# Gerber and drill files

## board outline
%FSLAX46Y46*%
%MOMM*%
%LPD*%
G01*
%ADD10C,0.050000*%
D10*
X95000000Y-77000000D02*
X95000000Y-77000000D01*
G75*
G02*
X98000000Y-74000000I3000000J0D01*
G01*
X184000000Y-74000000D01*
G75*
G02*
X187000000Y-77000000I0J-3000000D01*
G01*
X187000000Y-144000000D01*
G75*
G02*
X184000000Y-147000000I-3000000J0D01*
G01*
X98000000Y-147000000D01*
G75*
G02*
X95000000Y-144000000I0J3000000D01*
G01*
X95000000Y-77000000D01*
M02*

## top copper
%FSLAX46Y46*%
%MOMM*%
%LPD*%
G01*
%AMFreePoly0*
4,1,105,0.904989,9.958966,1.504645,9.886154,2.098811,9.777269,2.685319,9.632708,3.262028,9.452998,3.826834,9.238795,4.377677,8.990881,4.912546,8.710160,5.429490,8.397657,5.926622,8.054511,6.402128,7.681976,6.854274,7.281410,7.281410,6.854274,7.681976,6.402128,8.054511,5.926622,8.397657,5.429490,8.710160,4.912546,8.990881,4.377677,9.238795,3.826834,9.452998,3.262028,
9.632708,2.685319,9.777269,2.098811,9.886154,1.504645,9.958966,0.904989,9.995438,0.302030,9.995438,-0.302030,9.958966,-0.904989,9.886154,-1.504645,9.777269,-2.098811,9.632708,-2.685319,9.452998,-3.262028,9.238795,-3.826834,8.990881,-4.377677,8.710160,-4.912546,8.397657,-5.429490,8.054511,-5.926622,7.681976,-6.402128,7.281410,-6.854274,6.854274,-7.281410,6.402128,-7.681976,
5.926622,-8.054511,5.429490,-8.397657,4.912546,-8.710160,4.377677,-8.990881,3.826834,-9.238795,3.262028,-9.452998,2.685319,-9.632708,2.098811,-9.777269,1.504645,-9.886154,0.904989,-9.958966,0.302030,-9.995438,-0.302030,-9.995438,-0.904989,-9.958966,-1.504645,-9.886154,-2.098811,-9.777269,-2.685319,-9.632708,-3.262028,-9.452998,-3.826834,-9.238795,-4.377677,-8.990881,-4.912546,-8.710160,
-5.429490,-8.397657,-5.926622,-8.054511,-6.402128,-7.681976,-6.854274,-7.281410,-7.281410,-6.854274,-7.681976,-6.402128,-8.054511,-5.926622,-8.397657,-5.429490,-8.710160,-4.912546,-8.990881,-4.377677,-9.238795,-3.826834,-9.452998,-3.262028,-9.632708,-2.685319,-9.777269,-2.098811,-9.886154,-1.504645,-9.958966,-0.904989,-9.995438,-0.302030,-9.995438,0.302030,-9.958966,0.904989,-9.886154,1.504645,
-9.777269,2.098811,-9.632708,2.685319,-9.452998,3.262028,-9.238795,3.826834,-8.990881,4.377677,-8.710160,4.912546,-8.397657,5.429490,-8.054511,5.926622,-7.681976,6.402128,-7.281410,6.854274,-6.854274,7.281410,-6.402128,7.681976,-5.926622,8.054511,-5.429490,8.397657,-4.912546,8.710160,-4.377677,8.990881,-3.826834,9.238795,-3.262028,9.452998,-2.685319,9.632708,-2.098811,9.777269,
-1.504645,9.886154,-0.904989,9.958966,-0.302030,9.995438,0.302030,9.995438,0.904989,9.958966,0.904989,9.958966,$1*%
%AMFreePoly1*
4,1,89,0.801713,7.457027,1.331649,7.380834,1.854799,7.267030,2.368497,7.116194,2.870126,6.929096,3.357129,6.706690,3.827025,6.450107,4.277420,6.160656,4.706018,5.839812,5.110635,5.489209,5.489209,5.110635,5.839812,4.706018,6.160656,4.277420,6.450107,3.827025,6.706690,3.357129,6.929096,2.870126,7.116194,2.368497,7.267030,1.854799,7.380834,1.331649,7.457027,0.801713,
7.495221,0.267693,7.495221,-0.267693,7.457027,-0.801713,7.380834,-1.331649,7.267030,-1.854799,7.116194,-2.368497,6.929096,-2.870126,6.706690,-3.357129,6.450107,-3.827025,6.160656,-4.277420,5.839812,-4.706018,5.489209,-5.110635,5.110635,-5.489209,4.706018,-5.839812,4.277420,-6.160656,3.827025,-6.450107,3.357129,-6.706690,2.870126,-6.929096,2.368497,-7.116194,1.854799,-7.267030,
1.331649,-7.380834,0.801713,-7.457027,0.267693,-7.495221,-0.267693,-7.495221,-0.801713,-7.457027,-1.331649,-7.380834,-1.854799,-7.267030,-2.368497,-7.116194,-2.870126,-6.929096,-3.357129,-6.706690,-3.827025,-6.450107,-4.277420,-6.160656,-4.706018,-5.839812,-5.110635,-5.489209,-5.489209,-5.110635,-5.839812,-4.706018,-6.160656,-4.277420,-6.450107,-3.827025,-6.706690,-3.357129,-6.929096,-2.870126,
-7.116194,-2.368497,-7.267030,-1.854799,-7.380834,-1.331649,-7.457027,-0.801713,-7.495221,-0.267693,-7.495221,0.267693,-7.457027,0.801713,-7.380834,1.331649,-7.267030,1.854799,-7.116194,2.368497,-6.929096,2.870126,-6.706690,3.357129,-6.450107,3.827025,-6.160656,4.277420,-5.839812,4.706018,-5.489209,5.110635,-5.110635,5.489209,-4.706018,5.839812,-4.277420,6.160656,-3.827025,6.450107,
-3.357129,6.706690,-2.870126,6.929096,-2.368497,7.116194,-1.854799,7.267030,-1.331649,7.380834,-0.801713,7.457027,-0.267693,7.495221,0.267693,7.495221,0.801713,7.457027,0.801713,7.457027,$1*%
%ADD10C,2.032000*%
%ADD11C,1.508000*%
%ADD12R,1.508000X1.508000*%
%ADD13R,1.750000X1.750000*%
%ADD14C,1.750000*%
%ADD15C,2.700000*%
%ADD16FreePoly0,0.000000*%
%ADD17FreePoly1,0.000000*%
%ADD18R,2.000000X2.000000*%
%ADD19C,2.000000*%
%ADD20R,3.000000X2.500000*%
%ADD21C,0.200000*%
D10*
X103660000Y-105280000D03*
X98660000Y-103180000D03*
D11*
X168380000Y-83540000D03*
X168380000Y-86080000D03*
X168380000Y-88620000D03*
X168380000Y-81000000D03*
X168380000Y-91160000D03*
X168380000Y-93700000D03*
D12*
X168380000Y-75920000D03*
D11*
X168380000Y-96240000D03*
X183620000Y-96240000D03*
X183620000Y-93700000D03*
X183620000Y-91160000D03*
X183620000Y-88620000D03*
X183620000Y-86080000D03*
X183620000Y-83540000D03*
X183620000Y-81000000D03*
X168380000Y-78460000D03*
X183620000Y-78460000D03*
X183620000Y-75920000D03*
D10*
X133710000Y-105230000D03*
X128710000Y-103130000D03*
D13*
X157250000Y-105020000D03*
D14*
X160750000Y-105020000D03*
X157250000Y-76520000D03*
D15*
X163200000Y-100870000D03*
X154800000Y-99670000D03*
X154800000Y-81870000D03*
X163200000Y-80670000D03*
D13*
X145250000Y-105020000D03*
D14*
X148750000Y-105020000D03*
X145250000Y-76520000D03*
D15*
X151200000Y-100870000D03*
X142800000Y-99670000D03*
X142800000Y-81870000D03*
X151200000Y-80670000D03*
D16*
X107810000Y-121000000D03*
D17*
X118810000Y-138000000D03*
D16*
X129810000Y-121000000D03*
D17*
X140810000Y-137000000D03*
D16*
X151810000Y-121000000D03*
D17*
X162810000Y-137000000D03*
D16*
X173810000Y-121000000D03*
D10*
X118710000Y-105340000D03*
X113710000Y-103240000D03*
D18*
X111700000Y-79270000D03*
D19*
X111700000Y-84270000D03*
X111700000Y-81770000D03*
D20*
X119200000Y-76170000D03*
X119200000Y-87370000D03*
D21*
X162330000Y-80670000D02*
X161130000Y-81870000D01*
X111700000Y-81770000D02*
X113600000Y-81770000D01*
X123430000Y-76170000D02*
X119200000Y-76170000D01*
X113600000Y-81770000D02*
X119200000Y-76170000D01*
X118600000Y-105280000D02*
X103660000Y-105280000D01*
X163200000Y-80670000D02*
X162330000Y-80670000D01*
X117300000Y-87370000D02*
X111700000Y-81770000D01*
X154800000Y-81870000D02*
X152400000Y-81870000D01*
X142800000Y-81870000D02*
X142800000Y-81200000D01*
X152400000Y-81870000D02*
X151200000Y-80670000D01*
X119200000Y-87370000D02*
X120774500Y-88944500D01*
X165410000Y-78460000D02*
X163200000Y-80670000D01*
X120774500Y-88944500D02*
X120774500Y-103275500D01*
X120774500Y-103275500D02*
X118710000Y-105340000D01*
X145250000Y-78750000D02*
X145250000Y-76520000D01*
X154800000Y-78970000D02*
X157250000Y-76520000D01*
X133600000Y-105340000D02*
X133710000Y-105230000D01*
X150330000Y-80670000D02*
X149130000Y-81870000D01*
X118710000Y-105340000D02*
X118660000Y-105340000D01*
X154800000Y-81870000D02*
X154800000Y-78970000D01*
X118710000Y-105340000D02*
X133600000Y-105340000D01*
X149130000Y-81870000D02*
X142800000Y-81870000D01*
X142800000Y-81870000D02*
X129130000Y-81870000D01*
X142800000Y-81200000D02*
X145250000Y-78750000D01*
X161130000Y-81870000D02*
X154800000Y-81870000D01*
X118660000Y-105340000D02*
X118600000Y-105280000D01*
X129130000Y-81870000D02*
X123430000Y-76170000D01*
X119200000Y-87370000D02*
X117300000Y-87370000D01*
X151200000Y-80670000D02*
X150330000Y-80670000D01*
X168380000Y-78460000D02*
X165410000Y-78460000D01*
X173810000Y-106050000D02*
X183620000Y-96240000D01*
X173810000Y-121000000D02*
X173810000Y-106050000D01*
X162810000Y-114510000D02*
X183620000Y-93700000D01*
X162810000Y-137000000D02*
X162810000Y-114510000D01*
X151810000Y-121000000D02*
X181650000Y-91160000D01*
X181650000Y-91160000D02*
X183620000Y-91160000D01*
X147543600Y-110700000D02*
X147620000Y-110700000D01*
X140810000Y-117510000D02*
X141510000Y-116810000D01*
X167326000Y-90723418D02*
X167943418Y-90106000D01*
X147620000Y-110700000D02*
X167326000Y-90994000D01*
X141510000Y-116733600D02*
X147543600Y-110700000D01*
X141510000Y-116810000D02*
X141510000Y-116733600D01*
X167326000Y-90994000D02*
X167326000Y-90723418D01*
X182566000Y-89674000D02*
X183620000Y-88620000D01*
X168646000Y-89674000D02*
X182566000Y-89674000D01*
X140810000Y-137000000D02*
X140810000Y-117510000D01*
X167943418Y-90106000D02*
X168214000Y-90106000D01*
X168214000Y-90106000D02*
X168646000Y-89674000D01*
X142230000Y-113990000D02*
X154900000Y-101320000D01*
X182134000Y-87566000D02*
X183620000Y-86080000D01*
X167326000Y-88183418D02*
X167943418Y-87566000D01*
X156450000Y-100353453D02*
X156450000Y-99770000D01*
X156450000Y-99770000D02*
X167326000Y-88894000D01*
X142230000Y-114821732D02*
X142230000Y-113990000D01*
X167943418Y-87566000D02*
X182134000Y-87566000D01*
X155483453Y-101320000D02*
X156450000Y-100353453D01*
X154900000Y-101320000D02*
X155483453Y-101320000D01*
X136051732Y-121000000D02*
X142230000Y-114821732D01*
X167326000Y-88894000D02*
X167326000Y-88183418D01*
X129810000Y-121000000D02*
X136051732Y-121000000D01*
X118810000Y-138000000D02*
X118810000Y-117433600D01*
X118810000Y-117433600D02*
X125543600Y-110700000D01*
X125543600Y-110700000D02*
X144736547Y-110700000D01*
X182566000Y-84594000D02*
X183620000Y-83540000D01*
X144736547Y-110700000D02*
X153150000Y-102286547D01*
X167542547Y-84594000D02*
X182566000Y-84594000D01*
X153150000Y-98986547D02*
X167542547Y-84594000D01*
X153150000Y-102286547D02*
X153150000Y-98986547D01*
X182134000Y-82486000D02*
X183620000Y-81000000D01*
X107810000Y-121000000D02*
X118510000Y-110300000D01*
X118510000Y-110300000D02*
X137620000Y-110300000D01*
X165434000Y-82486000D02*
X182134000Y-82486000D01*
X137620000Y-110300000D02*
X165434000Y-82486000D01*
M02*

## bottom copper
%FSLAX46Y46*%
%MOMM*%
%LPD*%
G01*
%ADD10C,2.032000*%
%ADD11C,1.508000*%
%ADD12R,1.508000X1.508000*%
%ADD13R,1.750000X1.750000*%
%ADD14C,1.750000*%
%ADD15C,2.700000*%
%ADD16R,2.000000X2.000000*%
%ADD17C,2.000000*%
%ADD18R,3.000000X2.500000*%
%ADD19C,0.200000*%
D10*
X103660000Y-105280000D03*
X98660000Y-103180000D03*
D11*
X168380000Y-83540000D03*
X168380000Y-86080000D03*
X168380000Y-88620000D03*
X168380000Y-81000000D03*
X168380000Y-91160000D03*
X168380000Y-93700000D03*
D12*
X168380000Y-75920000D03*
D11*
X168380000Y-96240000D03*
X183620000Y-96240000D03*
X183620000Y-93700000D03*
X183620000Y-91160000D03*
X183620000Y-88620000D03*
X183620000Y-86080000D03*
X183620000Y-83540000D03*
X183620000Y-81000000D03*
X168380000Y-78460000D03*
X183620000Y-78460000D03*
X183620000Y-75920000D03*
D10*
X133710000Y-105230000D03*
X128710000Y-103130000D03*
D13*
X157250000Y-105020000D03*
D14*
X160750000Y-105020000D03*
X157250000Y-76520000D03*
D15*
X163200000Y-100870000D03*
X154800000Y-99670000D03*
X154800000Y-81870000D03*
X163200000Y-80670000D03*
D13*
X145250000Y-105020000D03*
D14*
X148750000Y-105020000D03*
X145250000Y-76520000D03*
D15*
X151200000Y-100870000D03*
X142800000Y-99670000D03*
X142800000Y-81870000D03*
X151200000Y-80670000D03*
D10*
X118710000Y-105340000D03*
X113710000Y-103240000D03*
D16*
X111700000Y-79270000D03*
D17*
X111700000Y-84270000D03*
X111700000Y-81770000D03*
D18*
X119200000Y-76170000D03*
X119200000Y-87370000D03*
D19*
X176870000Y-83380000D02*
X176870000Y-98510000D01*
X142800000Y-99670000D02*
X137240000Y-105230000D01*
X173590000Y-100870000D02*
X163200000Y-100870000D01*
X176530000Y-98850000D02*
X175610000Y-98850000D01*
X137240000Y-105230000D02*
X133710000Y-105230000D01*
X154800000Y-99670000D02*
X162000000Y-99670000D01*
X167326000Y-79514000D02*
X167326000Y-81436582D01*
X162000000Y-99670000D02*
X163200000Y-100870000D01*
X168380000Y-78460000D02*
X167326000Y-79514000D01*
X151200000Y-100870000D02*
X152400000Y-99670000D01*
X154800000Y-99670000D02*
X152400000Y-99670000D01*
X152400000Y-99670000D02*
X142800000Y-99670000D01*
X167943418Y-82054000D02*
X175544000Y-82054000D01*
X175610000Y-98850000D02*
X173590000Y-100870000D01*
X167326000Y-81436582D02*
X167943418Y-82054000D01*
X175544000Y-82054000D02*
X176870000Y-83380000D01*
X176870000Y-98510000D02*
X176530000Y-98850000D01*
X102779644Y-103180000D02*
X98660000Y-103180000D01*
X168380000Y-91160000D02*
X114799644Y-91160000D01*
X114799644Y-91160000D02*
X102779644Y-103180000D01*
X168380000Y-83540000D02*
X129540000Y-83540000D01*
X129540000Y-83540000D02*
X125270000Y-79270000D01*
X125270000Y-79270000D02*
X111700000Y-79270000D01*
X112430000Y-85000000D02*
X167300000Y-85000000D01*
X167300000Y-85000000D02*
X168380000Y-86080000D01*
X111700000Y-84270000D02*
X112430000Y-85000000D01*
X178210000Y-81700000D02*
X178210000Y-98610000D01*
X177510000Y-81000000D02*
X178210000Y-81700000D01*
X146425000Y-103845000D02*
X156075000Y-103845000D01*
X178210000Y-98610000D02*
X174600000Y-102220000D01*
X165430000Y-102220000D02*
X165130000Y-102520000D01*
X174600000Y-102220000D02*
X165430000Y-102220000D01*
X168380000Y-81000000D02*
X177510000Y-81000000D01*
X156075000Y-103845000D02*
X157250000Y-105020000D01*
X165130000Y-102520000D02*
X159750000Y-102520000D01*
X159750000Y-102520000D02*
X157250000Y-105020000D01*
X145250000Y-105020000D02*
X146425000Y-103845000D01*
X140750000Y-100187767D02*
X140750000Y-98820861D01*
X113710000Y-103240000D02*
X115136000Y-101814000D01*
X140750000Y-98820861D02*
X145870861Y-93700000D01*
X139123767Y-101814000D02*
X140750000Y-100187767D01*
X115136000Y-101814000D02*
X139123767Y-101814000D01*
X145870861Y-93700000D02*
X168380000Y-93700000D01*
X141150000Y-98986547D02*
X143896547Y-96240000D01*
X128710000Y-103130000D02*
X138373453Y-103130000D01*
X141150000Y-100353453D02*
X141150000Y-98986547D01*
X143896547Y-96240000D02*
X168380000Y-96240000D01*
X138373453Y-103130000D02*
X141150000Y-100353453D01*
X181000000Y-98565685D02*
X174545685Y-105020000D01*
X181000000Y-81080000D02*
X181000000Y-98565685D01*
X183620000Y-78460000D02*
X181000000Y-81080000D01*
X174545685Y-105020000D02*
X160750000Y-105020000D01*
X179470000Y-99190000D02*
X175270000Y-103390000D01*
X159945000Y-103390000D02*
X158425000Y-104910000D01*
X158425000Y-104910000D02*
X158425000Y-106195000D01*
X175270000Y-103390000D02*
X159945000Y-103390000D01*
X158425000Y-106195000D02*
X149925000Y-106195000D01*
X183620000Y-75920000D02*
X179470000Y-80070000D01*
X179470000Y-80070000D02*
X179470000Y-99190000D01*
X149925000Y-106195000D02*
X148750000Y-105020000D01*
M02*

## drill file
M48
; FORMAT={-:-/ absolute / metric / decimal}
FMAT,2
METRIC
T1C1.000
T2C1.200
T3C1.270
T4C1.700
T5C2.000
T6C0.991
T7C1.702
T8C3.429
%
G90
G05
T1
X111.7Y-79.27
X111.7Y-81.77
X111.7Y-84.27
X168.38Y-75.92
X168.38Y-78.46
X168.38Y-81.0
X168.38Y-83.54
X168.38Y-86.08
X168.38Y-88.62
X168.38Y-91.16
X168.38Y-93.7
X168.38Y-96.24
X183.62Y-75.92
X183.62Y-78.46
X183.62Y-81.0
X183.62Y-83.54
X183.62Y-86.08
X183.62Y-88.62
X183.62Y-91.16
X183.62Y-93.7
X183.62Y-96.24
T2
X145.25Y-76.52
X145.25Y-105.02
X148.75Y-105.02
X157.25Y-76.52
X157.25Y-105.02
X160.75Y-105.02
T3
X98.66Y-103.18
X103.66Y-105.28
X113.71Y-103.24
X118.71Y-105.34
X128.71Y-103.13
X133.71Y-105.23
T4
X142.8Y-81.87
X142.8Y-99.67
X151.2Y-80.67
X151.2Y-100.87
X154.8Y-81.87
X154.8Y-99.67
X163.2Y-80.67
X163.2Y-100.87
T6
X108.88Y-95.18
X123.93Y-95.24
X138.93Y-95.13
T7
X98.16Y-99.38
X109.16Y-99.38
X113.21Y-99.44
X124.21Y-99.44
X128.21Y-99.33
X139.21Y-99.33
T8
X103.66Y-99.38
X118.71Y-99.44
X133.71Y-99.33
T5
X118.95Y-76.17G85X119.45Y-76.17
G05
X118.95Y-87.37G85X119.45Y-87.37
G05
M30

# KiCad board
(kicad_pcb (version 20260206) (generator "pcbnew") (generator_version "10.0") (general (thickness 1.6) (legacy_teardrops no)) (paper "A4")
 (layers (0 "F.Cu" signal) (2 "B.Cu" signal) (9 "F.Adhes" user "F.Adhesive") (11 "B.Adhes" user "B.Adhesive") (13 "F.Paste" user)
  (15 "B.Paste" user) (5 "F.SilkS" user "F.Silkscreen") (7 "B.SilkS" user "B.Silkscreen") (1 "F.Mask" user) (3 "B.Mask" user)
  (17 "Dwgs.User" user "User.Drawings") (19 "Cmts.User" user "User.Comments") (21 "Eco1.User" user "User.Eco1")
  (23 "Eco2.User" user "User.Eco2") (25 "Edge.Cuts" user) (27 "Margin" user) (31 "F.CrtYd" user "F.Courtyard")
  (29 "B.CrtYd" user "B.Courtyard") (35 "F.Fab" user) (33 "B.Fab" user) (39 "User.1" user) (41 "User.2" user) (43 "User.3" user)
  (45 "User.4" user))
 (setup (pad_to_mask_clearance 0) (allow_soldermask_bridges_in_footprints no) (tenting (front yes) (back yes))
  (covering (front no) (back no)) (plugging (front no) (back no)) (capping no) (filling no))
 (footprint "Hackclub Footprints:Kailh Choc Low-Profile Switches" (layer "F.Cu") (at 103.66 99.38)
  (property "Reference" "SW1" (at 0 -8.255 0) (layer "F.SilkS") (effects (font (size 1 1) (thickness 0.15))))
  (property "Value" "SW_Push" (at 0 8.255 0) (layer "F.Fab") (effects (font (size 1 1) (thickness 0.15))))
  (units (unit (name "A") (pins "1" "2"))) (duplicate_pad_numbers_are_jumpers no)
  (pad "" np_thru_hole circle (at -5.5 0) (size 1.7018 1.7018) (drill 1.7018) (layers "*.Cu" "*.Mask"))
  (pad "" np_thru_hole circle (at 0 0) (size 3.429 3.429) (drill 3.429) (layers "*.Cu" "*.Mask"))
  (pad "" np_thru_hole circle (at 5.22 -4.2) (size 0.9906 0.9906) (drill 0.9906) (layers "*.Cu" "*.Mask"))
  (pad "" np_thru_hole circle (at 5.5 0) (size 1.7018 1.7018) (drill 1.7018) (layers "*.Cu" "*.Mask"))
  (pad "1" thru_hole circle (at 0 5.9) (size 2.032 2.032) (drill 1.27) (layers "*.Cu" "*.Mask") (remove_unused_layers no) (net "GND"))
  (pad "2" thru_hole circle (at -5 3.8) (size 2.032 2.032) (drill 1.27) (layers "*.Cu" "*.Mask") (remove_unused_layers no) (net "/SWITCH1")))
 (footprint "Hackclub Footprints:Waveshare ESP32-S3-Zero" (layer "F.Cu") (at 176 86.08)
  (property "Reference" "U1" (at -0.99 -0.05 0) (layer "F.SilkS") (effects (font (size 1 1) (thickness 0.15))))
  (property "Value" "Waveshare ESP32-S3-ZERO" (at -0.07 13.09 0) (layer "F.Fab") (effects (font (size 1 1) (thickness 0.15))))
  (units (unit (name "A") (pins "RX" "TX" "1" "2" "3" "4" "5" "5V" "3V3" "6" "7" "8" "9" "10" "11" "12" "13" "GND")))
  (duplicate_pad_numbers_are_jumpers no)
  (pad "1" thru_hole circle (at -7.62 -2.54) (size 1.508 1.508) (drill 1) (layers "*.Cu" "*.Mask") (remove_unused_layers no) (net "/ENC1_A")
   (solder_mask_margin 0.102))
  (pad "2" thru_hole circle (at -7.62 0) (size 1.508 1.508) (drill 1) (layers "*.Cu" "*.Mask") (remove_unused_layers no) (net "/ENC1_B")
   (solder_mask_margin 0.102))
  (pad "3" thru_hole circle (at -7.62 2.54) (size 1.508 1.508) (drill 1) (layers "*.Cu" "*.Mask") (remove_unused_layers no)
   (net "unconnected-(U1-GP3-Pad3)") (solder_mask_margin 0.102))
  (pad "3V3" thru_hole circle (at -7.62 -5.08) (size 1.508 1.508) (drill 1) (layers "*.Cu" "*.Mask") (remove_unused_layers no) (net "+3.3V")
   (solder_mask_margin 0.102))
  (pad "4" thru_hole circle (at -7.62 5.08) (size 1.508 1.508) (drill 1) (layers "*.Cu" "*.Mask") (remove_unused_layers no) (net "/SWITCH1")
   (solder_mask_margin 0.102))
  (pad "5" thru_hole circle (at -7.62 7.62) (size 1.508 1.508) (drill 1) (layers "*.Cu" "*.Mask") (remove_unused_layers no) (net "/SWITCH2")
   (solder_mask_margin 0.102))
  (pad "5V" thru_hole rect (at -7.62 -10.16) (size 1.508 1.508) (drill 1) (layers "*.Cu" "*.Mask") (remove_unused_layers no) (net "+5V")
   (solder_mask_margin 0.102))
  (pad "6" thru_hole circle (at -7.62 10.16) (size 1.508 1.508) (drill 1) (layers "*.Cu" "*.Mask") (remove_unused_layers no)
   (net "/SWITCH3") (solder_mask_margin 0.102))
  (pad "7" thru_hole circle (at 7.62 10.16) (size 1.508 1.508) (drill 1) (layers "*.Cu" "*.Mask") (remove_unused_layers no) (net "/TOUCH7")
   (solder_mask_margin 0.102))
  (pad "8" thru_hole circle (at 7.62 7.62) (size 1.508 1.508) (drill 1) (layers "*.Cu" "*.Mask") (remove_unused_layers no) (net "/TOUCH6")
   (solder_mask_margin 0.102))
  (pad "9" thru_hole circle (at 7.62 5.08) (size 1.508 1.508) (drill 1) (layers "*.Cu" "*.Mask") (remove_unused_layers no) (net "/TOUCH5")
   (solder_mask_margin 0.102))
  (pad "10" thru_hole circle (at 7.62 2.54) (size 1.508 1.508) (drill 1) (layers "*.Cu" "*.Mask") (remove_unused_layers no) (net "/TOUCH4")
   (solder_mask_margin 0.102))
  (pad "11" thru_hole circle (at 7.62 0) (size 1.508 1.508) (drill 1) (layers "*.Cu" "*.Mask") (remove_unused_layers no) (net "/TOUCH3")
   (solder_mask_margin 0.102))
  (pad "12" thru_hole circle (at 7.62 -2.54) (size 1.508 1.508) (drill 1) (layers "*.Cu" "*.Mask") (remove_unused_layers no) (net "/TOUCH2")
   (solder_mask_margin 0.102))
  (pad "13" thru_hole circle (at 7.62 -5.08) (size 1.508 1.508) (drill 1) (layers "*.Cu" "*.Mask") (remove_unused_layers no) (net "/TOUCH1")
   (solder_mask_margin 0.102))
  (pad "GND" thru_hole circle (at -7.62 -7.62) (size 1.508 1.508) (drill 1) (layers "*.Cu" "*.Mask") (remove_unused_layers no) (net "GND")
   (solder_mask_margin 0.102))
  (pad "RX" thru_hole circle (at 7.62 -7.62) (size 1.508 1.508) (drill 1) (layers "*.Cu" "*.Mask") (remove_unused_layers no)
   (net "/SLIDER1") (solder_mask_margin 0.102))
  (pad "TX" thru_hole circle (at 7.62 -10.16) (size 1.508 1.508) (drill 1) (layers "*.Cu" "*.Mask") (remove_unused_layers no)
   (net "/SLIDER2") (solder_mask_margin 0.102)))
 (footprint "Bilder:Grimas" (layer "F.Cu") (at 102.615412 81.967533)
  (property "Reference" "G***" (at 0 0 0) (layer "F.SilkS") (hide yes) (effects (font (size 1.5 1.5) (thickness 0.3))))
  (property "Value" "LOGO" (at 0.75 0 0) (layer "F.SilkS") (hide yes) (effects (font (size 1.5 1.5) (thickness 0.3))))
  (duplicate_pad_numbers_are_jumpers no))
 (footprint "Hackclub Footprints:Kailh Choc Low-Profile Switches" (layer "F.Cu") (at 133.71 99.33)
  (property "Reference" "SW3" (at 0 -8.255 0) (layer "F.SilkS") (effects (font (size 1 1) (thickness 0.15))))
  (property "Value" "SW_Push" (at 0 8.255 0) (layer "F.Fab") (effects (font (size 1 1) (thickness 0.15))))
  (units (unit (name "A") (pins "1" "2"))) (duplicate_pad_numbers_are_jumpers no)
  (pad "" np_thru_hole circle (at -5.5 0) (size 1.7018 1.7018) (drill 1.7018) (layers "*.Cu" "*.Mask"))
  (pad "" np_thru_hole circle (at 0 0) (size 3.429 3.429) (drill 3.429) (layers "*.Cu" "*.Mask"))
  (pad "" np_thru_hole circle (at 5.22 -4.2) (size 0.9906 0.9906) (drill 0.9906) (layers "*.Cu" "*.Mask"))
  (pad "" np_thru_hole circle (at 5.5 0) (size 1.7018 1.7018) (drill 1.7018) (layers "*.Cu" "*.Mask"))
  (pad "1" thru_hole circle (at 0 5.9) (size 2.032 2.032) (drill 1.27) (layers "*.Cu" "*.Mask") (remove_unused_layers no) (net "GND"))
  (pad "2" thru_hole circle (at -5 3.8) (size 2.032 2.032) (drill 1.27) (layers "*.Cu" "*.Mask") (remove_unused_layers no) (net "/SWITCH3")))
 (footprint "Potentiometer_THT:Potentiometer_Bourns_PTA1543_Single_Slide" (layer "F.Cu") (at 157.25 105.02 90)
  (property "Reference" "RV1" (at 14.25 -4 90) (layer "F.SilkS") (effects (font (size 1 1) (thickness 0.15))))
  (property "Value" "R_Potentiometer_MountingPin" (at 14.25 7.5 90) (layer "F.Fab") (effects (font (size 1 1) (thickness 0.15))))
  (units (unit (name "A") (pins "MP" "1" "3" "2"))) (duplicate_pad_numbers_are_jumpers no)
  (pad "1" thru_hole rect (at 0 0 90) (size 1.75 1.75) (drill 1.2) (layers "*.Cu" "*.Mask") (remove_unused_layers no) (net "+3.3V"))
  (pad "2" thru_hole circle (at 0 3.5 90) (size 1.75 1.75) (drill 1.2) (layers "*.Cu" "*.Mask") (remove_unused_layers no) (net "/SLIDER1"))
  (pad "3" thru_hole circle (at 28.5 0 90) (size 1.75 1.75) (drill 1.2) (layers "*.Cu" "*.Mask") (remove_unused_layers no) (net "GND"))
  (pad "MP" thru_hole circle (at 4.15 5.95 90) (size 2.7 2.7) (drill 1.7) (layers "*.Cu" "*.Mask") (remove_unused_layers no) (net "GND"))
  (pad "MP" thru_hole circle (at 5.35 -2.45 90) (size 2.7 2.7) (drill 1.7) (layers "*.Cu" "*.Mask") (remove_unused_layers no) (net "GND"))
  (pad "MP" thru_hole circle (at 23.15 -2.45 90) (size 2.7 2.7) (drill 1.7) (layers "*.Cu" "*.Mask") (remove_unused_layers no) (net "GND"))
  (pad "MP" thru_hole circle (at 24.35 5.95 90) (size 2.7 2.7) (drill 1.7) (layers "*.Cu" "*.Mask") (remove_unused_layers no) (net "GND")))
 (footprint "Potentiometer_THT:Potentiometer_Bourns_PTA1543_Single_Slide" (layer "F.Cu") (at 145.25 105.02 90)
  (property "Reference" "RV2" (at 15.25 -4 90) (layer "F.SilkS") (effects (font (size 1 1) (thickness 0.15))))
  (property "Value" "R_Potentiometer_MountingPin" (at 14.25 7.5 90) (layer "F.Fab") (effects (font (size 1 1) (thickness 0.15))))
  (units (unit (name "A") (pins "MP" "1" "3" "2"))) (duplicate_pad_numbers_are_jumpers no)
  (pad "1" thru_hole rect (at 0 0 90) (size 1.75 1.75) (drill 1.2) (layers "*.Cu" "*.Mask") (remove_unused_layers no) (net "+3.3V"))
  (pad "2" thru_hole circle (at 0 3.5 90) (size 1.75 1.75) (drill 1.2) (layers "*.Cu" "*.Mask") (remove_unused_layers no) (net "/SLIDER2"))
  (pad "3" thru_hole circle (at 28.5 0 90) (size 1.75 1.75) (drill 1.2) (layers "*.Cu" "*.Mask") (remove_unused_layers no) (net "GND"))
  (pad "MP" thru_hole circle (at 4.15 5.95 90) (size 2.7 2.7) (drill 1.7) (layers "*.Cu" "*.Mask") (remove_unused_layers no) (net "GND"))
  (pad "MP" thru_hole circle (at 5.35 -2.45 90) (size 2.7 2.7) (drill 1.7) (layers "*.Cu" "*.Mask") (remove_unused_layers no) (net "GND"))
  (pad "MP" thru_hole circle (at 23.15 -2.45 90) (size 2.7 2.7) (drill 1.7) (layers "*.Cu" "*.Mask") (remove_unused_layers no) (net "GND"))
  (pad "MP" thru_hole circle (at 24.35 5.95 90) (size 2.7 2.7) (drill 1.7) (layers "*.Cu" "*.Mask") (remove_unused_layers no) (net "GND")))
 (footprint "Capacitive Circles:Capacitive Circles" (layer "F.Cu") (at 140.81 109)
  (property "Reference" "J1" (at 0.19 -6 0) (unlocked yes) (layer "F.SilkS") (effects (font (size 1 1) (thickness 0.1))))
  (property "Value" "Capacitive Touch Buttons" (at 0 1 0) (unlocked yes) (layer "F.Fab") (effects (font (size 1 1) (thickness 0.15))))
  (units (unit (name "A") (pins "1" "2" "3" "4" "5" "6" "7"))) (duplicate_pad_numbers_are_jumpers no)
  (pad "1" smd custom (at -33 12) (size 20 20) (layers "F.Cu" "F.Mask") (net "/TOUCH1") (thermal_bridge_angle 90)
   (options (clearance outline) (anchor circle)) (primitives))
  (pad "2" smd custom (at -22 29) (size 15 15) (layers "F.Cu" "F.Mask") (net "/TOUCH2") (thermal_bridge_angle 90)
   (options (clearance outline) (anchor circle)) (primitives))
  (pad "3" smd custom (at -11 12) (size 20 20) (layers "F.Cu" "F.Mask") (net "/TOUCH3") (zone_connect 2) (thermal_bridge_angle 90)
   (options (clearance outline) (anchor circle)) (primitives))
  (pad "4" smd custom (at 0 28) (size 15 15) (layers "F.Cu" "F.Mask") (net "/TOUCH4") (zone_connect 2) (thermal_bridge_angle 90)
   (options (clearance outline) (anchor circle)) (primitives))
  (pad "5" smd custom (at 11 12) (size 20 20) (layers "F.Cu" "F.Mask") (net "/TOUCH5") (zone_connect 2) (thermal_bridge_angle 90)
   (options (clearance outline) (anchor circle)) (primitives))
  (pad "6" smd custom (at 22 28) (size 15 15) (layers "F.Cu" "F.Mask") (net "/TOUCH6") (zone_connect 2) (thermal_bridge_angle 90)
   (options (clearance outline) (anchor circle)) (primitives))
  (pad "7" smd custom (at 33 12) (size 20 20) (layers "F.Cu" "F.Mask") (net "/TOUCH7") (zone_connect 2) (thermal_bridge_angle 90)
   (options (clearance outline) (anchor circle)) (primitives)))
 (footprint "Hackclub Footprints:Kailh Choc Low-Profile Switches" (layer "F.Cu") (at 118.71 99.44)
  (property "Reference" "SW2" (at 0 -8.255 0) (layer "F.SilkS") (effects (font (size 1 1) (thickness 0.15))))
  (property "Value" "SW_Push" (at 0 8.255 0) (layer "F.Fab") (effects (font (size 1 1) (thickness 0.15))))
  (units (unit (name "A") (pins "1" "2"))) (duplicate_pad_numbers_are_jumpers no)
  (pad "" np_thru_hole circle (at -5.5 0) (size 1.7018 1.7018) (drill 1.7018) (layers "*.Cu" "*.Mask"))
  (pad "" np_thru_hole circle (at 0 0) (size 3.429 3.429) (drill 3.429) (layers "*.Cu" "*.Mask"))
  (pad "" np_thru_hole circle (at 5.22 -4.2) (size 0.9906 0.9906) (drill 0.9906) (layers "*.Cu" "*.Mask"))
  (pad "" np_thru_hole circle (at 5.5 0) (size 1.7018 1.7018) (drill 1.7018) (layers "*.Cu" "*.Mask"))
  (pad "1" thru_hole circle (at 0 5.9) (size 2.032 2.032) (drill 1.27) (layers "*.Cu" "*.Mask") (remove_unused_layers no) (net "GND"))
  (pad "2" thru_hole circle (at -5 3.8) (size 2.032 2.032) (drill 1.27) (layers "*.Cu" "*.Mask") (remove_unused_layers no) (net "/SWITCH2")))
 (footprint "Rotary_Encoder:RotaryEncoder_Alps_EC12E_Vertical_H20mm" (layer "F.Cu") (at 111.7 79.27)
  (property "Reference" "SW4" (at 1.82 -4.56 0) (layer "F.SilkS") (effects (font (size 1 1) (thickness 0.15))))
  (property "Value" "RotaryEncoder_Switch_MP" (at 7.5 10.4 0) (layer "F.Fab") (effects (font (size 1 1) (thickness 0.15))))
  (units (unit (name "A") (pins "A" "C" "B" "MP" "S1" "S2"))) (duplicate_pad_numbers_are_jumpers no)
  (pad "A" thru_hole rect (at 0 0) (size 2 2) (drill 1) (layers "*.Cu" "*.Mask") (remove_unused_layers no) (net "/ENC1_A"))
  (pad "B" thru_hole circle (at 0 5) (size 2 2) (drill 1) (layers "*.Cu" "*.Mask") (remove_unused_layers no) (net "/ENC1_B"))
  (pad "C" thru_hole circle (at 0 2.5) (size 2 2) (drill 1) (layers "*.Cu" "*.Mask") (remove_unused_layers no) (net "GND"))
  (pad "MP" thru_hole rect (at 7.5 -3.1) (size 3 2.5) (drill oval 2.5 2) (layers "*.Cu" "*.Mask") (remove_unused_layers no) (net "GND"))
  (pad "MP" thru_hole rect (at 7.5 8.1) (size 3 2.5) (drill oval 2.5 2) (layers "*.Cu" "*.Mask") (remove_unused_layers no) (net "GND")))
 (gr_rect (start 95 74) (end 187 147) (radius 3) (stroke (width 0.05) (type solid)) (fill no) (layer "Edge.Cuts"))
 (segment (start 162.33 80.67) (end 161.13 81.87) (width 0.2) (layer "F.Cu") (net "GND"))
 (segment (start 111.7 81.77) (end 113.6 81.77) (width 0.2) (layer "F.Cu") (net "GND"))
 (segment (start 123.43 76.17) (end 119.2 76.17) (width 0.2) (layer "F.Cu") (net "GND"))
 (segment (start 113.6 81.77) (end 119.2 76.17) (width 0.2) (layer "F.Cu") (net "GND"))
 (segment (start 118.6 105.28) (end 103.66 105.28) (width 0.2) (layer "F.Cu") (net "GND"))
 (segment (start 163.2 80.67) (end 162.33 80.67) (width 0.2) (layer "F.Cu") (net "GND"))
 (segment (start 117.3 87.37) (end 111.7 81.77) (width 0.2) (layer "F.Cu") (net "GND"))
 (segment (start 154.8 81.87) (end 152.4 81.87) (width 0.2) (layer "F.Cu") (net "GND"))
 (segment (start 142.8 81.87) (end 142.8 81.2) (width 0.2) (layer "F.Cu") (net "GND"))
 (segment (start 152.4 81.87) (end 151.2 80.67) (width 0.2) (layer "F.Cu") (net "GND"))
 (segment (start 119.2 87.37) (end 120.7745 88.9445) (width 0.2) (layer "F.Cu") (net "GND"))
 (segment (start 165.41 78.46) (end 163.2 80.67) (width 0.2) (layer "F.Cu") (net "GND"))
 (segment (start 120.7745 88.9445) (end 120.7745 103.2755) (width 0.2) (layer "F.Cu") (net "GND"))
 (segment (start 120.7745 103.2755) (end 118.71 105.34) (width 0.2) (layer "F.Cu") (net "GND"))
 (segment (start 145.25 78.75) (end 145.25 76.52) (width 0.2) (layer "F.Cu") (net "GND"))
 (segment (start 154.8 78.97) (end 157.25 76.52) (width 0.2) (layer "F.Cu") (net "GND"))
 (segment (start 133.6 105.34) (end 133.71 105.23) (width 0.2) (layer "F.Cu") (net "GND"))
 (segment (start 150.33 80.67) (end 149.13 81.87) (width 0.2) (layer "F.Cu") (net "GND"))
 (segment (start 118.71 105.34) (end 118.66 105.34) (width 0.2) (layer "F.Cu") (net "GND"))
 (segment (start 154.8 81.87) (end 154.8 78.97) (width 0.2) (layer "F.Cu") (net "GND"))
 (segment (start 118.71 105.34) (end 133.6 105.34) (width 0.2) (layer "F.Cu") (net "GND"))
 (segment (start 149.13 81.87) (end 142.8 81.87) (width 0.2) (layer "F.Cu") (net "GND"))
 (segment (start 142.8 81.87) (end 129.13 81.87) (width 0.2) (layer "F.Cu") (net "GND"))
 (segment (start 142.8 81.2) (end 145.25 78.75) (width 0.2) (layer "F.Cu") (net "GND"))
 (segment (start 161.13 81.87) (end 154.8 81.87) (width 0.2) (layer "F.Cu") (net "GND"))
 (segment (start 118.66 105.34) (end 118.6 105.28) (width 0.2) (layer "F.Cu") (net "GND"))
 (segment (start 129.13 81.87) (end 123.43 76.17) (width 0.2) (layer "F.Cu") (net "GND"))
 (segment (start 119.2 87.37) (end 117.3 87.37) (width 0.2) (layer "F.Cu") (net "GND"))
 (segment (start 151.2 80.67) (end 150.33 80.67) (width 0.2) (layer "F.Cu") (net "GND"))
 (segment (start 168.38 78.46) (end 165.41 78.46) (width 0.2) (layer "F.Cu") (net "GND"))
 (segment (start 176.87 83.38) (end 176.87 98.51) (width 0.2) (layer "B.Cu") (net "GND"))
 (segment (start 142.8 99.67) (end 137.24 105.23) (width 0.2) (layer "B.Cu") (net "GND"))
 (segment (start 173.59 100.87) (end 163.2 100.87) (width 0.2) (layer "B.Cu") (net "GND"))
 (segment (start 176.53 98.85) (end 175.61 98.85) (width 0.2) (layer "B.Cu") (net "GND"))
 (segment (start 137.24 105.23) (end 133.71 105.23) (width 0.2) (layer "B.Cu") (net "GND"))
 (segment (start 154.8 99.67) (end 162 99.67) (width 0.2) (layer "B.Cu") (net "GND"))
 (segment (start 167.326 79.514) (end 167.326 81.436582) (width 0.2) (layer "B.Cu") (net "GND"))
 (segment (start 162 99.67) (end 163.2 100.87) (width 0.2) (layer "B.Cu") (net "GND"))
 (segment (start 168.38 78.46) (end 167.326 79.514) (width 0.2) (layer "B.Cu") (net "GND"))
 (segment (start 151.2 100.87) (end 152.4 99.67) (width 0.2) (layer "B.Cu") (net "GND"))
 (segment (start 154.8 99.67) (end 152.4 99.67) (width 0.2) (layer "B.Cu") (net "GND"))
 (segment (start 152.4 99.67) (end 142.8 99.67) (width 0.2) (layer "B.Cu") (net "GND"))
 (segment (start 167.943418 82.054) (end 175.544 82.054) (width 0.2) (layer "B.Cu") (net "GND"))
 (segment (start 175.61 98.85) (end 173.59 100.87) (width 0.2) (layer "B.Cu") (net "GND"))
 (segment (start 167.326 81.436582) (end 167.943418 82.054) (width 0.2) (layer "B.Cu") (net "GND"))
 (segment (start 175.544 82.054) (end 176.87 83.38) (width 0.2) (layer "B.Cu") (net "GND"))
 (segment (start 176.87 98.51) (end 176.53 98.85) (width 0.2) (layer "B.Cu") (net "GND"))
 (segment (start 102.779644 103.18) (end 98.66 103.18) (width 0.2) (layer "B.Cu") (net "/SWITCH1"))
 (segment (start 168.38 91.16) (end 114.799644 91.16) (width 0.2) (layer "B.Cu") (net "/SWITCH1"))
 (segment (start 114.799644 91.16) (end 102.779644 103.18) (width 0.2) (layer "B.Cu") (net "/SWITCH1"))
 (segment (start 168.38 83.54) (end 129.54 83.54) (width 0.2) (layer "B.Cu") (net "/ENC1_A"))
 (segment (start 129.54 83.54) (end 125.27 79.27) (width 0.2) (layer "B.Cu") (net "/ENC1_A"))
 (segment (start 125.27 79.27) (end 111.7 79.27) (width 0.2) (layer "B.Cu") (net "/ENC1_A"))
 (segment (start 112.43 85) (end 167.3 85) (width 0.2) (layer "B.Cu") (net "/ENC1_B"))
 (segment (start 167.3 85) (end 168.38 86.08) (width 0.2) (layer "B.Cu") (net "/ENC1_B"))
 (segment (start 111.7 84.27) (end 112.43 85) (width 0.2) (layer "B.Cu") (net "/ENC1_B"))
 (segment (start 178.21 81.7) (end 178.21 98.61) (width 0.2) (layer "B.Cu") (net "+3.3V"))
 (segment (start 177.51 81) (end 178.21 81.7) (width 0.2) (layer "B.Cu") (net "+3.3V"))
 (segment (start 146.425 103.845) (end 156.075 103.845) (width 0.2) (layer "B.Cu") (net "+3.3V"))
 (segment (start 178.21 98.61) (end 174.6 102.22) (width 0.2) (layer "B.Cu") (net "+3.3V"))
 (segment (start 165.43 102.22) (end 165.13 102.52) (width 0.2) (layer "B.Cu") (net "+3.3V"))
 (segment (start 174.6 102.22) (end 165.43 102.22) (width 0.2) (layer "B.Cu") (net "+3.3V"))
 (segment (start 168.38 81) (end 177.51 81) (width 0.2) (layer "B.Cu") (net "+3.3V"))
 (segment (start 156.075 103.845) (end 157.25 105.02) (width 0.2) (layer "B.Cu") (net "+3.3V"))
 (segment (start 165.13 102.52) (end 159.75 102.52) (width 0.2) (layer "B.Cu") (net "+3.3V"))
 (segment (start 159.75 102.52) (end 157.25 105.02) (width 0.2) (layer "B.Cu") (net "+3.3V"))
 (segment (start 145.25 105.02) (end 146.425 103.845) (width 0.2) (layer "B.Cu") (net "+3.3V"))
 (segment (start 140.75 100.187767) (end 140.75 98.820861) (width 0.2) (layer "B.Cu") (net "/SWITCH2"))
 (segment (start 113.71 103.24) (end 115.136 101.814) (width 0.2) (layer "B.Cu") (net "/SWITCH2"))
 (segment (start 140.75 98.820861) (end 145.870861 93.7) (width 0.2) (layer "B.Cu") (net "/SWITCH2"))
 (segment (start 139.123767 101.814) (end 140.75 100.187767) (width 0.2) (layer "B.Cu") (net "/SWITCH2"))
 (segment (start 115.136 101.814) (end 139.123767 101.814) (width 0.2) (layer "B.Cu") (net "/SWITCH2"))
 (segment (start 145.870861 93.7) (end 168.38 93.7) (width 0.2) (layer "B.Cu") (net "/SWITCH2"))
 (segment (start 141.15 98.986547) (end 143.896547 96.24) (width 0.2) (layer "B.Cu") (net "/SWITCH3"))
 (segment (start 128.71 103.13) (end 138.373453 103.13) (width 0.2) (layer "B.Cu") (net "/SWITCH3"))
 (segment (start 141.15 100.353453) (end 141.15 98.986547) (width 0.2) (layer "B.Cu") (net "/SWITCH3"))
 (segment (start 143.896547 96.24) (end 168.38 96.24) (width 0.2) (layer "B.Cu") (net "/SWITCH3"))
 (segment (start 138.373453 103.13) (end 141.15 100.353453) (width 0.2) (layer "B.Cu") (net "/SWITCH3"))
 (segment (start 173.81 106.05) (end 183.62 96.24) (width 0.2) (layer "F.Cu") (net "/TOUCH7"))
 (segment (start 173.81 121) (end 173.81 106.05) (width 0.2) (layer "F.Cu") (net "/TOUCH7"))
 (segment (start 162.81 114.51) (end 183.62 93.7) (width 0.2) (layer "F.Cu") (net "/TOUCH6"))
 (segment (start 162.81 137) (end 162.81 114.51) (width 0.2) (layer "F.Cu") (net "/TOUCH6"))
 (segment (start 151.81 121) (end 181.65 91.16) (width 0.2) (layer "F.Cu") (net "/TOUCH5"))
 (segment (start 181.65 91.16) (end 183.62 91.16) (width 0.2) (layer "F.Cu") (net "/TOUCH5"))
 (segment (start 147.5436 110.7) (end 147.62 110.7) (width 0.2) (layer "F.Cu") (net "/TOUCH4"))
 (segment (start 140.81 117.51) (end 141.51 116.81) (width 0.2) (layer "F.Cu") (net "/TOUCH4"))
 (segment (start 167.326 90.723418) (end 167.943418 90.106) (width 0.2) (layer "F.Cu") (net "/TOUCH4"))
 (segment (start 147.62 110.7) (end 167.326 90.994) (width 0.2) (layer "F.Cu") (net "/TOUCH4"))
 (segment (start 141.51 116.7336) (end 147.5436 110.7) (width 0.2) (layer "F.Cu") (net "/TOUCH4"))
 (segment (start 141.51 116.81) (end 141.51 116.7336) (width 0.2) (layer "F.Cu") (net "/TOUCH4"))
 (segment (start 167.326 90.994) (end 167.326 90.723418) (width 0.2) (layer "F.Cu") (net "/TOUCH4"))
 (segment (start 182.566 89.674) (end 183.62 88.62) (width 0.2) (layer "F.Cu") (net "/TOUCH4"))
 (segment (start 168.646 89.674) (end 182.566 89.674) (width 0.2) (layer "F.Cu") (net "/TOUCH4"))
 (segment (start 140.81 137) (end 140.81 117.51) (width 0.2) (layer "F.Cu") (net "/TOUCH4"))
 (segment (start 167.943418 90.106) (end 168.214 90.106) (width 0.2) (layer "F.Cu") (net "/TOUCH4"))
 (segment (start 168.214 90.106) (end 168.646 89.674) (width 0.2) (layer "F.Cu") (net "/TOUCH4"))
 (segment (start 142.23 113.99) (end 154.9 101.32) (width 0.2) (layer "F.Cu") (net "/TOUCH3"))
 (segment (start 182.134 87.566) (end 183.62 86.08) (width 0.2) (layer "F.Cu") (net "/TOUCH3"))
 (segment (start 167.326 88.183418) (end 167.943418 87.566) (width 0.2) (layer "F.Cu") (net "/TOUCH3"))
 (segment (start 156.45 100.353453) (end 156.45 99.77) (width 0.2) (layer "F.Cu") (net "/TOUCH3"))
 (segment (start 156.45 99.77) (end 167.326 88.894) (width 0.2) (layer "F.Cu") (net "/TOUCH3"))
 (segment (start 142.23 114.821732) (end 142.23 113.99) (width 0.2) (layer "F.Cu") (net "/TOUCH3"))
 (segment (start 167.943418 87.566) (end 182.134 87.566) (width 0.2) (layer "F.Cu") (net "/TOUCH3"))
 (segment (start 155.483453 101.32) (end 156.45 100.353453) (width 0.2) (layer "F.Cu") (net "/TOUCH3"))
 (segment (start 154.9 101.32) (end 155.483453 101.32) (width 0.2) (layer "F.Cu") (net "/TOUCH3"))
 (segment (start 136.051732 121) (end 142.23 114.821732) (width 0.2) (layer "F.Cu") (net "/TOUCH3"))
 (segment (start 167.326 88.894) (end 167.326 88.183418) (width 0.2) (layer "F.Cu") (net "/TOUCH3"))
 (segment (start 129.81 121) (end 136.051732 121) (width 0.2) (layer "F.Cu") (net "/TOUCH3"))
 (segment (start 118.81 138) (end 118.81 117.4336) (width 0.2) (layer "F.Cu") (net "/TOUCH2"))
 (segment (start 118.81 117.4336) (end 125.5436 110.7) (width 0.2) (layer "F.Cu") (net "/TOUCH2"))
 (segment (start 125.5436 110.7) (end 144.736547 110.7) (width 0.2) (layer "F.Cu") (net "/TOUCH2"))
 (segment (start 182.566 84.594) (end 183.62 83.54) (width 0.2) (layer "F.Cu") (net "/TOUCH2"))
 (segment (start 144.736547 110.7) (end 153.15 102.286547) (width 0.2) (layer "F.Cu") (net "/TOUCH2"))
 (segment (start 167.542547 84.594) (end 182.566 84.594) (width 0.2) (layer "F.Cu") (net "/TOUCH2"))
 (segment (start 153.15 98.986547) (end 167.542547 84.594) (width 0.2) (layer "F.Cu") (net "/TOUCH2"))
 (segment (start 153.15 102.286547) (end 153.15 98.986547) (width 0.2) (layer "F.Cu") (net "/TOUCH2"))
 (segment (start 182.134 82.486) (end 183.62 81) (width 0.2) (layer "F.Cu") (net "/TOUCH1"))
 (segment (start 107.81 121) (end 118.51 110.3) (width 0.2) (layer "F.Cu") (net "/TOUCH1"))
 (segment (start 118.51 110.3) (end 137.62 110.3) (width 0.2) (layer "F.Cu") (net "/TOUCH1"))
 (segment (start 165.434 82.486) (end 182.134 82.486) (width 0.2) (layer "F.Cu") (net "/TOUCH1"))
 (segment (start 137.62 110.3) (end 165.434 82.486) (width 0.2) (layer "F.Cu") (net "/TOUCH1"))
 (segment (start 181 98.565685) (end 174.545685 105.02) (width 0.2) (layer "B.Cu") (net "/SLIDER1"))
 (segment (start 181 81.08) (end 181 98.565685) (width 0.2) (layer "B.Cu") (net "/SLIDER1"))
 (segment (start 183.62 78.46) (end 181 81.08) (width 0.2) (layer "B.Cu") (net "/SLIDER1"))
 (segment (start 174.545685 105.02) (end 160.75 105.02) (width 0.2) (layer "B.Cu") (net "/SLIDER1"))
 (segment (start 179.47 99.19) (end 175.27 103.39) (width 0.2) (layer "B.Cu") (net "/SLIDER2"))
 (segment (start 159.945 103.39) (end 158.425 104.91) (width 0.2) (layer "B.Cu") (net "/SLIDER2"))
 (segment (start 158.425 104.91) (end 158.425 106.195) (width 0.2) (layer "B.Cu") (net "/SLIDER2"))
 (segment (start 175.27 103.39) (end 159.945 103.39) (width 0.2) (layer "B.Cu") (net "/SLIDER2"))
 (segment (start 158.425 106.195) (end 149.925 106.195) (width 0.2) (layer "B.Cu") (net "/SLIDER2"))
 (segment (start 183.62 75.92) (end 179.47 80.07) (width 0.2) (layer "B.Cu") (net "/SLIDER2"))
 (segment (start 179.47 80.07) (end 179.47 99.19) (width 0.2) (layer "B.Cu") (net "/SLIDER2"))
 (segment (start 149.925 106.195) (end 148.75 105.02) (width 0.2) (layer "B.Cu") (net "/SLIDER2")))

